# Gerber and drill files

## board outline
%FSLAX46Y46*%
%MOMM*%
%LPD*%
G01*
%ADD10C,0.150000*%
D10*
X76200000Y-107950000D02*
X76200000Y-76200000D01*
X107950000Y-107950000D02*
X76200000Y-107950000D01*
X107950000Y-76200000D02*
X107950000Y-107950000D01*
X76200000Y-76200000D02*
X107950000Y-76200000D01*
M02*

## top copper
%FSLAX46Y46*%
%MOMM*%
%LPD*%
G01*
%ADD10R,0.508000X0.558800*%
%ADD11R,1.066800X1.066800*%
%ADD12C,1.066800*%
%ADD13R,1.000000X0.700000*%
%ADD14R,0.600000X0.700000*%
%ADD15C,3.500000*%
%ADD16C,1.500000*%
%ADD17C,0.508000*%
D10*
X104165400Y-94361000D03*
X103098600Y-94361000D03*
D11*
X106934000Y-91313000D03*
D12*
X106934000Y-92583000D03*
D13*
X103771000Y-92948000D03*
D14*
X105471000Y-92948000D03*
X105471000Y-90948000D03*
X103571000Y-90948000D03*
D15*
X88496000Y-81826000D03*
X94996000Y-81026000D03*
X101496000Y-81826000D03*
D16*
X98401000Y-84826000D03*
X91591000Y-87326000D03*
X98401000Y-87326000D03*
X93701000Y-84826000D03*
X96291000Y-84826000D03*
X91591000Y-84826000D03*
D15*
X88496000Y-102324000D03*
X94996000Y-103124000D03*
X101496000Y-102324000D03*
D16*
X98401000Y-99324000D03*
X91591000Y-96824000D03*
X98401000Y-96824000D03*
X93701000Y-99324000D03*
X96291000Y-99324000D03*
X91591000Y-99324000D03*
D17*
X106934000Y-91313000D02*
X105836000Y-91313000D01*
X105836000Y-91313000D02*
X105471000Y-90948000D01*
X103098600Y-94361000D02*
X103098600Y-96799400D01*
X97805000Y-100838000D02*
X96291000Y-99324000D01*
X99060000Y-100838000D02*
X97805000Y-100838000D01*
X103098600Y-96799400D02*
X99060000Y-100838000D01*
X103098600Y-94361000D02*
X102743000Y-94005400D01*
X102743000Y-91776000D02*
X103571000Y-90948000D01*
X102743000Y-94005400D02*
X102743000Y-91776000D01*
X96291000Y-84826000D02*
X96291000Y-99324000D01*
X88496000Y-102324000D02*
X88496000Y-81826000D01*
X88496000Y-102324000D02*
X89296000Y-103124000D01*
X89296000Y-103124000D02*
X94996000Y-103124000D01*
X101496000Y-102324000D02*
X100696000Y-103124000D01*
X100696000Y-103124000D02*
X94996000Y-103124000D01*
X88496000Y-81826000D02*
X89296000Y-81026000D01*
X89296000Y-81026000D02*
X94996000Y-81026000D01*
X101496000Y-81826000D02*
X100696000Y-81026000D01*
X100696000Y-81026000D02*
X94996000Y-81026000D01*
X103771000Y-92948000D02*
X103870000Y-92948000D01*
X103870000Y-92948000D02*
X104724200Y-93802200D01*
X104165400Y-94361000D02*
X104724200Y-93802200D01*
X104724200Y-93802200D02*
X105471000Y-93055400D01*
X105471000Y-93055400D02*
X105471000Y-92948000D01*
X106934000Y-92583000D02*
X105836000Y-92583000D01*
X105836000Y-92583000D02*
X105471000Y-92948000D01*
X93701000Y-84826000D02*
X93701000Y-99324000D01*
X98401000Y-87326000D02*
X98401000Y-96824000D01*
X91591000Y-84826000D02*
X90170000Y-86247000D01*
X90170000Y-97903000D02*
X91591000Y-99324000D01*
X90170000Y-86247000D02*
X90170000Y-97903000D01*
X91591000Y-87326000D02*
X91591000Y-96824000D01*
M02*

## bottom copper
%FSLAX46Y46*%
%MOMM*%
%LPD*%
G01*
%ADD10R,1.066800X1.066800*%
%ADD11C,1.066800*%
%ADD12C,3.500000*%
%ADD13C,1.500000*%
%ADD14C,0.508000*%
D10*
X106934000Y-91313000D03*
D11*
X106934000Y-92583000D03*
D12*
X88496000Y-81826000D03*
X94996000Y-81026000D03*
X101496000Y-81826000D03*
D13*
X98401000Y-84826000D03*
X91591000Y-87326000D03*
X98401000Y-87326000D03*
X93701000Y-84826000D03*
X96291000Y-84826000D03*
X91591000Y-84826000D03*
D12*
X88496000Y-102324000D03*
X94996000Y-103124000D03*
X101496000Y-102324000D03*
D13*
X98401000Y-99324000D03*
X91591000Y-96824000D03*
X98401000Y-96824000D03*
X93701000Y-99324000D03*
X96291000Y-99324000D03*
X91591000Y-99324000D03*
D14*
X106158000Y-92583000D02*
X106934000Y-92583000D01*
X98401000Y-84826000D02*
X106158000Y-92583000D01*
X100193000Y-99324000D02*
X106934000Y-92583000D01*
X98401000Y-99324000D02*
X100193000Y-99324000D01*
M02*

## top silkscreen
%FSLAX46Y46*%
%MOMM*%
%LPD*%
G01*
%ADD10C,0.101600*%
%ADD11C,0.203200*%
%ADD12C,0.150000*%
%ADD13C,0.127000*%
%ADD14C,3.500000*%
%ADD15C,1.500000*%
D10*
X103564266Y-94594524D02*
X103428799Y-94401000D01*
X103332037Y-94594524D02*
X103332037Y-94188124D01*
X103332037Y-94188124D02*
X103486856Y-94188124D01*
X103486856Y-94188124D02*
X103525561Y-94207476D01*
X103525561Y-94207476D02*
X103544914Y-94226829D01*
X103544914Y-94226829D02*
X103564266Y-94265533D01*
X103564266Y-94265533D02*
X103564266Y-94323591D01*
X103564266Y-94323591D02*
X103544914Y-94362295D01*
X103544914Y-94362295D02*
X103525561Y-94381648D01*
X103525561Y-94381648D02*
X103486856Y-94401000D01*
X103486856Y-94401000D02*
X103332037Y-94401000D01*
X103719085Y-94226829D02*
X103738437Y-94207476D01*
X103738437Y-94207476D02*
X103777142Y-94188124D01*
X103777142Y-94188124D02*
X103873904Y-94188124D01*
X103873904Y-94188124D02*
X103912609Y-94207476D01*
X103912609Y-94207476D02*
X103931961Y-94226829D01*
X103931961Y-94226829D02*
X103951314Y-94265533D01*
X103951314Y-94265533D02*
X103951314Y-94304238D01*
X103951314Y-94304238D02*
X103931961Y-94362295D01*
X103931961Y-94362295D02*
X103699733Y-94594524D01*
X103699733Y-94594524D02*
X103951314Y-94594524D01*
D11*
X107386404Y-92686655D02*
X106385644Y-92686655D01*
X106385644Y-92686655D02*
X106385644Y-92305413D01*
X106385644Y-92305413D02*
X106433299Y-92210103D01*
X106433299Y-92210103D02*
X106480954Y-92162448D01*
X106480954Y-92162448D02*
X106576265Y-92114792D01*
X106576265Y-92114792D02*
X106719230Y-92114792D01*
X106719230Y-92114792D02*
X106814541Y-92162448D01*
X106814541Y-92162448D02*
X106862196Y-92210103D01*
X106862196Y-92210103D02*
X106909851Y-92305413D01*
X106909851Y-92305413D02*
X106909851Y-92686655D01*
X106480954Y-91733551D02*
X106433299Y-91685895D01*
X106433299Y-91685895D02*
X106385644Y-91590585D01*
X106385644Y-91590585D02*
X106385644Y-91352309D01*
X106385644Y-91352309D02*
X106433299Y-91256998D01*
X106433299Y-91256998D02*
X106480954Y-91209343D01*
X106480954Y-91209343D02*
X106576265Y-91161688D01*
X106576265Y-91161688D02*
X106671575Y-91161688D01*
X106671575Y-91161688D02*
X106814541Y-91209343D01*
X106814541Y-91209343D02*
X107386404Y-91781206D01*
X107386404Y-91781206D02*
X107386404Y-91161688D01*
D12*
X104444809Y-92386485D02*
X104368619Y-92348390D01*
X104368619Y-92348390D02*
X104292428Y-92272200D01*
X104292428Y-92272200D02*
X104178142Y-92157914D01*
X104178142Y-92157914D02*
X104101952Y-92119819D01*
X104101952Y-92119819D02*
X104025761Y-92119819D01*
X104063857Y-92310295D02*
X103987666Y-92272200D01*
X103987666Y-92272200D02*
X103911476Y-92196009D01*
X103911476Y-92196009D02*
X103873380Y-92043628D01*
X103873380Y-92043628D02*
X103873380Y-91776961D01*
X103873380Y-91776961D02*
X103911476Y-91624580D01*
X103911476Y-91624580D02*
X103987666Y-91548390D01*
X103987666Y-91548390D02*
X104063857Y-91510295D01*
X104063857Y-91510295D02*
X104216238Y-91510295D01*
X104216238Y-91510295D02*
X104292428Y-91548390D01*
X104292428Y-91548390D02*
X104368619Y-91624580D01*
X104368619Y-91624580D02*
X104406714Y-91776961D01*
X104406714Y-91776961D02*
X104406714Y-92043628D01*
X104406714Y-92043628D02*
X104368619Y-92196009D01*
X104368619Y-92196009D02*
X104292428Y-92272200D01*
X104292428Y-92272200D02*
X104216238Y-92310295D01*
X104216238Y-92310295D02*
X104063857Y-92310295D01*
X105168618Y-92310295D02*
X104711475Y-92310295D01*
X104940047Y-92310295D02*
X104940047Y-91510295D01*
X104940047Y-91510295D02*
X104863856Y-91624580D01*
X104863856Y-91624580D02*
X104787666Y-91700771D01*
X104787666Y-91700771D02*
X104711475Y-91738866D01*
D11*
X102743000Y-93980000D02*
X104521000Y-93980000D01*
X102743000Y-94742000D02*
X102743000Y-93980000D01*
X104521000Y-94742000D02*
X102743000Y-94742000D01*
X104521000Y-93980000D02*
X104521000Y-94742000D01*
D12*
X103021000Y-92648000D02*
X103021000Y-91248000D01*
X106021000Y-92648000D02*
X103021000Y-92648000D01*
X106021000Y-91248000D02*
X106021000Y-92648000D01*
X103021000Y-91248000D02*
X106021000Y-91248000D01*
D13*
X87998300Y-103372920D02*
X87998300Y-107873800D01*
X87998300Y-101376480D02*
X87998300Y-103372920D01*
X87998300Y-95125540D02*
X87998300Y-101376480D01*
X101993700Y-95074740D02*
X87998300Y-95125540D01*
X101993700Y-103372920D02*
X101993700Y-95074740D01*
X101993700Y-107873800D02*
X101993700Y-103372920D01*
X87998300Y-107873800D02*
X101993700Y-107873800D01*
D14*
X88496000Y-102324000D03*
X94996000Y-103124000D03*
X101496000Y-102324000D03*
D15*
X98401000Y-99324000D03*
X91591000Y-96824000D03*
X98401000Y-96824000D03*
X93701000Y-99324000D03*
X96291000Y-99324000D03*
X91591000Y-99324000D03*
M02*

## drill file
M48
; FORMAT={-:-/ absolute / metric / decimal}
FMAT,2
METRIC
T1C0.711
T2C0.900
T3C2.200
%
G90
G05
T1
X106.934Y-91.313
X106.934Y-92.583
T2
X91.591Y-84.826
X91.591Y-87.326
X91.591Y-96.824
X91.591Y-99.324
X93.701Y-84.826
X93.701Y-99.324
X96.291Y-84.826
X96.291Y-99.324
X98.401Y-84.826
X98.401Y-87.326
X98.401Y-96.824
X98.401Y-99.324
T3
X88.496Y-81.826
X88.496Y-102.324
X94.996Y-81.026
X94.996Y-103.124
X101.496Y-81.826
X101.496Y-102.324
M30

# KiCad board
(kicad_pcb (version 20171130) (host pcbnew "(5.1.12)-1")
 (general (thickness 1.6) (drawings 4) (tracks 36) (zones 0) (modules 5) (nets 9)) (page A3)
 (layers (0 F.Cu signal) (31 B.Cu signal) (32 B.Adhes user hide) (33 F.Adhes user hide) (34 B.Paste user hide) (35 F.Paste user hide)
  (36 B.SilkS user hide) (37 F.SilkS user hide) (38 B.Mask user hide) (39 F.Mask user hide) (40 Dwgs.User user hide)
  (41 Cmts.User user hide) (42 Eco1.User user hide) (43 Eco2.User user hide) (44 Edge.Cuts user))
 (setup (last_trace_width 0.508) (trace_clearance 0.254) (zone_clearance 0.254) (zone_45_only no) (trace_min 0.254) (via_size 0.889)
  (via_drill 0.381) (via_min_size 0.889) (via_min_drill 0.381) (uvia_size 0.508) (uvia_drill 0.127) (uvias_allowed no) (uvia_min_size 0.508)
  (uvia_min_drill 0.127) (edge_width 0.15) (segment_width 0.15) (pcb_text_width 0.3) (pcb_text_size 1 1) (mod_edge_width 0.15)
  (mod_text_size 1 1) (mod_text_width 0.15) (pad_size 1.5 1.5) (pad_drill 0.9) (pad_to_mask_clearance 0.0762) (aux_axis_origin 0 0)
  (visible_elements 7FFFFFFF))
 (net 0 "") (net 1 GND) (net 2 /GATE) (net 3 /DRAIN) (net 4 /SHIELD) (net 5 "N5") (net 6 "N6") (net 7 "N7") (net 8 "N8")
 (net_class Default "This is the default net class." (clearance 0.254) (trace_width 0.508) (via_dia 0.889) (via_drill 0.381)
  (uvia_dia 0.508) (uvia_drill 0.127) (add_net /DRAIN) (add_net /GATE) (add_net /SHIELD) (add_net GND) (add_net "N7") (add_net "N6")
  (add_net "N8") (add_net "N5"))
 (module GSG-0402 (layer F.Cu) (at 103.632 94.361) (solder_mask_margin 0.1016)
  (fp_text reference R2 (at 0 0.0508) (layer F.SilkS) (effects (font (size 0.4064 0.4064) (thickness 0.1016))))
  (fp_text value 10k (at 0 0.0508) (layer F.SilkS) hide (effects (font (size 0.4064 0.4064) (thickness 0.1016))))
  (fp_line (start -0.889 -0.381) (end 0.889 -0.381) (layer F.SilkS) (width 0.2032))
  (fp_line (start -0.889 0.381) (end -0.889 -0.381) (layer F.SilkS) (width 0.2032))
  (fp_line (start 0.889 0.381) (end -0.889 0.381) (layer F.SilkS) (width 0.2032))
  (fp_line (start 0.889 -0.381) (end 0.889 0.381) (layer F.SilkS) (width 0.2032))
  (pad 2 smd rect (at 0.5334 0) (size 0.508 0.5588) (layers F.Cu F.Paste F.Mask) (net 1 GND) (solder_mask_margin 0.1016))
  (pad 1 smd rect (at -0.5334 0) (size 0.508 0.5588) (layers F.Cu F.Paste F.Mask) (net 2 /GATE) (die_length -1518.485687)
   (solder_mask_margin 0.1016)))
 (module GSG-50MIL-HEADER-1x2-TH (layer F.Cu) (at 106.934 91.948 270)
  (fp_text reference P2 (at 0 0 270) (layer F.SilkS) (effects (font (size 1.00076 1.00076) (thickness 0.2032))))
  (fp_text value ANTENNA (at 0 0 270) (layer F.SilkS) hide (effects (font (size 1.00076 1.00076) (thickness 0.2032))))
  (pad 1 thru_hole rect (at -0.635 0 270) (size 1.0668 1.0668) (drill 0.7112) (layers *.Cu *.Mask) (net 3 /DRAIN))
  (pad 2 thru_hole circle (at 0.635 0 270) (size 1.0668 1.0668) (drill 0.7112) (layers *.Cu *.Mask) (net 1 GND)))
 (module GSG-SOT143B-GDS (layer F.Cu) (at 104.521 91.948)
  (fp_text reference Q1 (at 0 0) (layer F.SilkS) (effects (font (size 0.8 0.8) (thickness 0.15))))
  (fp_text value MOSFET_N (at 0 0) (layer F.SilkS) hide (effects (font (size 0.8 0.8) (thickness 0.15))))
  (fp_line (start -1.5 0.7) (end -1.5 -0.7) (layer F.SilkS) (width 0.15))
  (fp_line (start 1.5 0.7) (end -1.5 0.7) (layer F.SilkS) (width 0.15))
  (fp_line (start 1.5 -0.7) (end 1.5 0.7) (layer F.SilkS) (width 0.15))
  (fp_line (start -1.5 -0.7) (end 1.5 -0.7) (layer F.SilkS) (width 0.15))
  (pad B smd rect (at -0.75 1) (size 1 0.7) (layers F.Cu F.Paste F.Mask) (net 1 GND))
  (pad S smd rect (at 0.95 1) (size 0.6 0.7) (layers F.Cu F.Paste F.Mask) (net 1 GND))
  (pad D smd rect (at 0.95 -1) (size 0.6 0.7) (layers F.Cu F.Paste F.Mask) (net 3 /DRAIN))
  (pad G smd rect (at -0.95 -1) (size 0.6 0.7) (layers F.Cu F.Paste F.Mask) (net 2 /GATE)))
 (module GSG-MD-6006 (layer B.Cu) (at 94.996 81.026 180)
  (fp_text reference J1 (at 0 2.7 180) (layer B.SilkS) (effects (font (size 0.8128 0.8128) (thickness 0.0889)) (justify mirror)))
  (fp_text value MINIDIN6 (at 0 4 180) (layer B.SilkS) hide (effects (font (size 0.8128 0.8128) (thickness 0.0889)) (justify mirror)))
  (pad 0 thru_hole circle (at 6.5 -0.8 180) (size 3.5 3.5) (drill 2.2) (layers *.Cu *.Mask B.SilkS) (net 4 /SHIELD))
  (pad 0 thru_hole circle (at 0 0 180) (size 3.5 3.5) (drill 2.2) (layers *.Cu *.Mask B.SilkS) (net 4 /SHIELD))
  (pad 0 thru_hole circle (at -6.5 -0.8 180) (size 3.5 3.5) (drill 2.2) (layers *.Cu *.Mask B.SilkS) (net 4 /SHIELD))
  (pad 3 thru_hole circle (at -3.405 -3.8 180) (size 1.5 1.5) (drill 0.9) (layers *.Cu *.Mask B.SilkS) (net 1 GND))
  (pad 6 thru_hole circle (at 3.405 -6.3 180) (size 1.5 1.5) (drill 0.9) (layers *.Cu *.Mask B.SilkS) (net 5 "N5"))
  (pad 5 thru_hole circle (at -3.405 -6.3 180) (size 1.5 1.5) (drill 0.9) (layers *.Cu *.Mask B.SilkS) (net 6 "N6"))
  (pad 2 thru_hole circle (at 1.295 -3.8 180) (size 1.5 1.5) (drill 0.9) (layers *.Cu *.Mask B.SilkS) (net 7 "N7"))
  (pad 1 thru_hole circle (at -1.295 -3.8 180) (size 1.5 1.5) (drill 0.9) (layers *.Cu *.Mask B.SilkS) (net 2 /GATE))
  (pad 4 thru_hole circle (at 3.405 -3.8 180) (size 1.5 1.5) (drill 0.9) (layers *.Cu *.Mask B.SilkS) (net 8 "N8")))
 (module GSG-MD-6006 (layer F.Cu) (at 94.996 103.124 180)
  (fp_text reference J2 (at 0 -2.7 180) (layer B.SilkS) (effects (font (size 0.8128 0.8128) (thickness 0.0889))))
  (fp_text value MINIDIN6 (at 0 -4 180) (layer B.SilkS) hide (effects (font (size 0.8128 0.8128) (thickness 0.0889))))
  (fp_line (start 6.9977 -0.24892) (end 6.9977 -4.7498) (layer F.SilkS) (width 0.127))
  (fp_line (start 6.9977 1.74752) (end 6.9977 -0.24892) (layer F.SilkS) (width 0.127))
  (fp_line (start 6.9977 7.99846) (end 6.9977 1.74752) (layer F.SilkS) (width 0.127))
  (fp_line (start -6.9977 8.04926) (end 6.9977 7.99846) (layer F.SilkS) (width 0.127))
  (fp_line (start -6.9977 -0.24892) (end -6.9977 8.04926) (layer F.SilkS) (width 0.127))
  (fp_line (start -6.9977 -4.7498) (end -6.9977 -0.24892) (layer F.SilkS) (width 0.127))
  (fp_line (start 6.9977 -4.7498) (end -6.9977 -4.7498) (layer F.SilkS) (width 0.127))
  (pad 0 thru_hole circle (at 6.5 0.8 180) (size 3.5 3.5) (drill 2.2) (layers *.Cu *.Mask F.SilkS) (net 4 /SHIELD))
  (pad 0 thru_hole circle (at 0 0 180) (size 3.5 3.5) (drill 2.2) (layers *.Cu *.Mask F.SilkS) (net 4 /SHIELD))
  (pad 0 thru_hole circle (at -6.5 0.8 180) (size 3.5 3.5) (drill 2.2) (layers *.Cu *.Mask F.SilkS) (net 4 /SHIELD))
  (pad 3 thru_hole circle (at -3.405 3.8 180) (size 1.5 1.5) (drill 0.9) (layers *.Cu *.Mask F.SilkS) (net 1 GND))
  (pad 6 thru_hole circle (at 3.405 6.3 180) (size 1.5 1.5) (drill 0.9) (layers *.Cu *.Mask F.SilkS) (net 5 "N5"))
  (pad 5 thru_hole circle (at -3.405 6.3 180) (size 1.5 1.5) (drill 0.9) (layers *.Cu *.Mask F.SilkS) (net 6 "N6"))
  (pad 2 thru_hole circle (at 1.295 3.8 180) (size 1.5 1.5) (drill 0.9) (layers *.Cu *.Mask F.SilkS) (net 7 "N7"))
  (pad 1 thru_hole circle (at -1.295 3.8 180) (size 1.5 1.5) (drill 0.9) (layers *.Cu *.Mask F.SilkS) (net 2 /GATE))
  (pad 4 thru_hole circle (at 3.405 3.8 180) (size 1.5 1.5) (drill 0.9) (layers *.Cu *.Mask F.SilkS) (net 8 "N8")))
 (gr_line (start 76.2 107.95) (end 76.2 76.2) (angle 90) (layer Edge.Cuts) (width 0.15))
 (gr_line (start 107.95 107.95) (end 76.2 107.95) (angle 90) (layer Edge.Cuts) (width 0.15))
 (gr_line (start 107.95 76.2) (end 107.95 107.95) (angle 90) (layer Edge.Cuts) (width 0.15))
 (gr_line (start 76.2 76.2) (end 107.95 76.2) (angle 90) (layer Edge.Cuts) (width 0.15))
 (segment (start 106.934 91.313) (end 105.836 91.313) (width 0.508) (layer F.Cu) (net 3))
 (segment (start 105.836 91.313) (end 105.471 90.948) (width 0.508) (layer F.Cu) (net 3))
 (segment (start 103.0986 94.361) (end 103.0986 96.7994) (width 0.508) (layer F.Cu) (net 2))
 (segment (start 97.805 100.838) (end 96.291 99.324) (width 0.508) (layer F.Cu) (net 2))
 (segment (start 99.06 100.838) (end 97.805 100.838) (width 0.508) (layer F.Cu) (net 2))
 (segment (start 103.0986 96.7994) (end 99.06 100.838) (width 0.508) (layer F.Cu) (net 2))
 (segment (start 103.0986 94.361) (end 102.743 94.0054) (width 0.508) (layer F.Cu) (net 2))
 (segment (start 102.743 91.776) (end 103.571 90.948) (width 0.508) (layer F.Cu) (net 2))
 (segment (start 102.743 94.0054) (end 102.743 91.776) (width 0.508) (layer F.Cu) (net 2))
 (segment (start 96.291 84.826) (end 96.291 99.324) (width 0.508) (layer F.Cu) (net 2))
 (segment (start 88.496 102.324) (end 88.496 81.826) (width 0.508) (layer F.Cu) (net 4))
 (segment (start 88.496 102.324) (end 89.296 103.124) (width 0.508) (layer F.Cu) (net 4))
 (segment (start 89.296 103.124) (end 94.996 103.124) (width 0.508) (layer F.Cu) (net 4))
 (segment (start 101.496 102.324) (end 100.696 103.124) (width 0.508) (layer F.Cu) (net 4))
 (segment (start 100.696 103.124) (end 94.996 103.124) (width 0.508) (layer F.Cu) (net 4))
 (segment (start 88.496 81.826) (end 89.296 81.026) (width 0.508) (layer F.Cu) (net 4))
 (segment (start 89.296 81.026) (end 94.996 81.026) (width 0.508) (layer F.Cu) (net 4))
 (segment (start 101.496 81.826) (end 100.696 81.026) (width 0.508) (layer F.Cu) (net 4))
 (segment (start 100.696 81.026) (end 94.996 81.026) (width 0.508) (layer F.Cu) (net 4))
 (segment (start 103.771 92.948) (end 103.87 92.948) (width 0.508) (layer F.Cu) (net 1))
 (segment (start 103.87 92.948) (end 104.7242 93.8022) (width 0.508) (layer F.Cu) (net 1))
 (segment (start 104.1654 94.361) (end 104.7242 93.8022) (width 0.508) (layer F.Cu) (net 1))
 (segment (start 104.7242 93.8022) (end 105.471 93.0554) (width 0.508) (layer F.Cu) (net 1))
 (segment (start 105.471 93.0554) (end 105.471 92.948) (width 0.508) (layer F.Cu) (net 1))
 (segment (start 106.934 92.583) (end 105.836 92.583) (width 0.508) (layer F.Cu) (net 1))
 (segment (start 105.836 92.583) (end 105.471 92.948) (width 0.508) (layer F.Cu) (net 1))
 (segment (start 106.158 92.583) (end 106.934 92.583) (width 0.508) (layer B.Cu) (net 1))
 (segment (start 98.401 84.826) (end 106.158 92.583) (width 0.508) (layer B.Cu) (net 1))
 (segment (start 100.193 99.324) (end 106.934 92.583) (width 0.508) (layer B.Cu) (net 1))
 (segment (start 98.401 99.324) (end 100.193 99.324) (width 0.508) (layer B.Cu) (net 1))
 (segment (start 93.701 84.826) (end 93.701 99.324) (width 0.508) (layer F.Cu) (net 7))
 (segment (start 98.401 87.326) (end 98.401 96.824) (width 0.508) (layer F.Cu) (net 6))
 (segment (start 91.591 84.826) (end 90.17 86.247) (width 0.508) (layer F.Cu) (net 8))
 (segment (start 90.17 97.903) (end 91.591 99.324) (width 0.508) (layer F.Cu) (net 8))
 (segment (start 90.17 86.247) (end 90.17 97.903) (width 0.508) (layer F.Cu) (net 8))
 (segment (start 91.591 87.326) (end 91.591 96.824) (width 0.508) (layer F.Cu) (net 5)))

